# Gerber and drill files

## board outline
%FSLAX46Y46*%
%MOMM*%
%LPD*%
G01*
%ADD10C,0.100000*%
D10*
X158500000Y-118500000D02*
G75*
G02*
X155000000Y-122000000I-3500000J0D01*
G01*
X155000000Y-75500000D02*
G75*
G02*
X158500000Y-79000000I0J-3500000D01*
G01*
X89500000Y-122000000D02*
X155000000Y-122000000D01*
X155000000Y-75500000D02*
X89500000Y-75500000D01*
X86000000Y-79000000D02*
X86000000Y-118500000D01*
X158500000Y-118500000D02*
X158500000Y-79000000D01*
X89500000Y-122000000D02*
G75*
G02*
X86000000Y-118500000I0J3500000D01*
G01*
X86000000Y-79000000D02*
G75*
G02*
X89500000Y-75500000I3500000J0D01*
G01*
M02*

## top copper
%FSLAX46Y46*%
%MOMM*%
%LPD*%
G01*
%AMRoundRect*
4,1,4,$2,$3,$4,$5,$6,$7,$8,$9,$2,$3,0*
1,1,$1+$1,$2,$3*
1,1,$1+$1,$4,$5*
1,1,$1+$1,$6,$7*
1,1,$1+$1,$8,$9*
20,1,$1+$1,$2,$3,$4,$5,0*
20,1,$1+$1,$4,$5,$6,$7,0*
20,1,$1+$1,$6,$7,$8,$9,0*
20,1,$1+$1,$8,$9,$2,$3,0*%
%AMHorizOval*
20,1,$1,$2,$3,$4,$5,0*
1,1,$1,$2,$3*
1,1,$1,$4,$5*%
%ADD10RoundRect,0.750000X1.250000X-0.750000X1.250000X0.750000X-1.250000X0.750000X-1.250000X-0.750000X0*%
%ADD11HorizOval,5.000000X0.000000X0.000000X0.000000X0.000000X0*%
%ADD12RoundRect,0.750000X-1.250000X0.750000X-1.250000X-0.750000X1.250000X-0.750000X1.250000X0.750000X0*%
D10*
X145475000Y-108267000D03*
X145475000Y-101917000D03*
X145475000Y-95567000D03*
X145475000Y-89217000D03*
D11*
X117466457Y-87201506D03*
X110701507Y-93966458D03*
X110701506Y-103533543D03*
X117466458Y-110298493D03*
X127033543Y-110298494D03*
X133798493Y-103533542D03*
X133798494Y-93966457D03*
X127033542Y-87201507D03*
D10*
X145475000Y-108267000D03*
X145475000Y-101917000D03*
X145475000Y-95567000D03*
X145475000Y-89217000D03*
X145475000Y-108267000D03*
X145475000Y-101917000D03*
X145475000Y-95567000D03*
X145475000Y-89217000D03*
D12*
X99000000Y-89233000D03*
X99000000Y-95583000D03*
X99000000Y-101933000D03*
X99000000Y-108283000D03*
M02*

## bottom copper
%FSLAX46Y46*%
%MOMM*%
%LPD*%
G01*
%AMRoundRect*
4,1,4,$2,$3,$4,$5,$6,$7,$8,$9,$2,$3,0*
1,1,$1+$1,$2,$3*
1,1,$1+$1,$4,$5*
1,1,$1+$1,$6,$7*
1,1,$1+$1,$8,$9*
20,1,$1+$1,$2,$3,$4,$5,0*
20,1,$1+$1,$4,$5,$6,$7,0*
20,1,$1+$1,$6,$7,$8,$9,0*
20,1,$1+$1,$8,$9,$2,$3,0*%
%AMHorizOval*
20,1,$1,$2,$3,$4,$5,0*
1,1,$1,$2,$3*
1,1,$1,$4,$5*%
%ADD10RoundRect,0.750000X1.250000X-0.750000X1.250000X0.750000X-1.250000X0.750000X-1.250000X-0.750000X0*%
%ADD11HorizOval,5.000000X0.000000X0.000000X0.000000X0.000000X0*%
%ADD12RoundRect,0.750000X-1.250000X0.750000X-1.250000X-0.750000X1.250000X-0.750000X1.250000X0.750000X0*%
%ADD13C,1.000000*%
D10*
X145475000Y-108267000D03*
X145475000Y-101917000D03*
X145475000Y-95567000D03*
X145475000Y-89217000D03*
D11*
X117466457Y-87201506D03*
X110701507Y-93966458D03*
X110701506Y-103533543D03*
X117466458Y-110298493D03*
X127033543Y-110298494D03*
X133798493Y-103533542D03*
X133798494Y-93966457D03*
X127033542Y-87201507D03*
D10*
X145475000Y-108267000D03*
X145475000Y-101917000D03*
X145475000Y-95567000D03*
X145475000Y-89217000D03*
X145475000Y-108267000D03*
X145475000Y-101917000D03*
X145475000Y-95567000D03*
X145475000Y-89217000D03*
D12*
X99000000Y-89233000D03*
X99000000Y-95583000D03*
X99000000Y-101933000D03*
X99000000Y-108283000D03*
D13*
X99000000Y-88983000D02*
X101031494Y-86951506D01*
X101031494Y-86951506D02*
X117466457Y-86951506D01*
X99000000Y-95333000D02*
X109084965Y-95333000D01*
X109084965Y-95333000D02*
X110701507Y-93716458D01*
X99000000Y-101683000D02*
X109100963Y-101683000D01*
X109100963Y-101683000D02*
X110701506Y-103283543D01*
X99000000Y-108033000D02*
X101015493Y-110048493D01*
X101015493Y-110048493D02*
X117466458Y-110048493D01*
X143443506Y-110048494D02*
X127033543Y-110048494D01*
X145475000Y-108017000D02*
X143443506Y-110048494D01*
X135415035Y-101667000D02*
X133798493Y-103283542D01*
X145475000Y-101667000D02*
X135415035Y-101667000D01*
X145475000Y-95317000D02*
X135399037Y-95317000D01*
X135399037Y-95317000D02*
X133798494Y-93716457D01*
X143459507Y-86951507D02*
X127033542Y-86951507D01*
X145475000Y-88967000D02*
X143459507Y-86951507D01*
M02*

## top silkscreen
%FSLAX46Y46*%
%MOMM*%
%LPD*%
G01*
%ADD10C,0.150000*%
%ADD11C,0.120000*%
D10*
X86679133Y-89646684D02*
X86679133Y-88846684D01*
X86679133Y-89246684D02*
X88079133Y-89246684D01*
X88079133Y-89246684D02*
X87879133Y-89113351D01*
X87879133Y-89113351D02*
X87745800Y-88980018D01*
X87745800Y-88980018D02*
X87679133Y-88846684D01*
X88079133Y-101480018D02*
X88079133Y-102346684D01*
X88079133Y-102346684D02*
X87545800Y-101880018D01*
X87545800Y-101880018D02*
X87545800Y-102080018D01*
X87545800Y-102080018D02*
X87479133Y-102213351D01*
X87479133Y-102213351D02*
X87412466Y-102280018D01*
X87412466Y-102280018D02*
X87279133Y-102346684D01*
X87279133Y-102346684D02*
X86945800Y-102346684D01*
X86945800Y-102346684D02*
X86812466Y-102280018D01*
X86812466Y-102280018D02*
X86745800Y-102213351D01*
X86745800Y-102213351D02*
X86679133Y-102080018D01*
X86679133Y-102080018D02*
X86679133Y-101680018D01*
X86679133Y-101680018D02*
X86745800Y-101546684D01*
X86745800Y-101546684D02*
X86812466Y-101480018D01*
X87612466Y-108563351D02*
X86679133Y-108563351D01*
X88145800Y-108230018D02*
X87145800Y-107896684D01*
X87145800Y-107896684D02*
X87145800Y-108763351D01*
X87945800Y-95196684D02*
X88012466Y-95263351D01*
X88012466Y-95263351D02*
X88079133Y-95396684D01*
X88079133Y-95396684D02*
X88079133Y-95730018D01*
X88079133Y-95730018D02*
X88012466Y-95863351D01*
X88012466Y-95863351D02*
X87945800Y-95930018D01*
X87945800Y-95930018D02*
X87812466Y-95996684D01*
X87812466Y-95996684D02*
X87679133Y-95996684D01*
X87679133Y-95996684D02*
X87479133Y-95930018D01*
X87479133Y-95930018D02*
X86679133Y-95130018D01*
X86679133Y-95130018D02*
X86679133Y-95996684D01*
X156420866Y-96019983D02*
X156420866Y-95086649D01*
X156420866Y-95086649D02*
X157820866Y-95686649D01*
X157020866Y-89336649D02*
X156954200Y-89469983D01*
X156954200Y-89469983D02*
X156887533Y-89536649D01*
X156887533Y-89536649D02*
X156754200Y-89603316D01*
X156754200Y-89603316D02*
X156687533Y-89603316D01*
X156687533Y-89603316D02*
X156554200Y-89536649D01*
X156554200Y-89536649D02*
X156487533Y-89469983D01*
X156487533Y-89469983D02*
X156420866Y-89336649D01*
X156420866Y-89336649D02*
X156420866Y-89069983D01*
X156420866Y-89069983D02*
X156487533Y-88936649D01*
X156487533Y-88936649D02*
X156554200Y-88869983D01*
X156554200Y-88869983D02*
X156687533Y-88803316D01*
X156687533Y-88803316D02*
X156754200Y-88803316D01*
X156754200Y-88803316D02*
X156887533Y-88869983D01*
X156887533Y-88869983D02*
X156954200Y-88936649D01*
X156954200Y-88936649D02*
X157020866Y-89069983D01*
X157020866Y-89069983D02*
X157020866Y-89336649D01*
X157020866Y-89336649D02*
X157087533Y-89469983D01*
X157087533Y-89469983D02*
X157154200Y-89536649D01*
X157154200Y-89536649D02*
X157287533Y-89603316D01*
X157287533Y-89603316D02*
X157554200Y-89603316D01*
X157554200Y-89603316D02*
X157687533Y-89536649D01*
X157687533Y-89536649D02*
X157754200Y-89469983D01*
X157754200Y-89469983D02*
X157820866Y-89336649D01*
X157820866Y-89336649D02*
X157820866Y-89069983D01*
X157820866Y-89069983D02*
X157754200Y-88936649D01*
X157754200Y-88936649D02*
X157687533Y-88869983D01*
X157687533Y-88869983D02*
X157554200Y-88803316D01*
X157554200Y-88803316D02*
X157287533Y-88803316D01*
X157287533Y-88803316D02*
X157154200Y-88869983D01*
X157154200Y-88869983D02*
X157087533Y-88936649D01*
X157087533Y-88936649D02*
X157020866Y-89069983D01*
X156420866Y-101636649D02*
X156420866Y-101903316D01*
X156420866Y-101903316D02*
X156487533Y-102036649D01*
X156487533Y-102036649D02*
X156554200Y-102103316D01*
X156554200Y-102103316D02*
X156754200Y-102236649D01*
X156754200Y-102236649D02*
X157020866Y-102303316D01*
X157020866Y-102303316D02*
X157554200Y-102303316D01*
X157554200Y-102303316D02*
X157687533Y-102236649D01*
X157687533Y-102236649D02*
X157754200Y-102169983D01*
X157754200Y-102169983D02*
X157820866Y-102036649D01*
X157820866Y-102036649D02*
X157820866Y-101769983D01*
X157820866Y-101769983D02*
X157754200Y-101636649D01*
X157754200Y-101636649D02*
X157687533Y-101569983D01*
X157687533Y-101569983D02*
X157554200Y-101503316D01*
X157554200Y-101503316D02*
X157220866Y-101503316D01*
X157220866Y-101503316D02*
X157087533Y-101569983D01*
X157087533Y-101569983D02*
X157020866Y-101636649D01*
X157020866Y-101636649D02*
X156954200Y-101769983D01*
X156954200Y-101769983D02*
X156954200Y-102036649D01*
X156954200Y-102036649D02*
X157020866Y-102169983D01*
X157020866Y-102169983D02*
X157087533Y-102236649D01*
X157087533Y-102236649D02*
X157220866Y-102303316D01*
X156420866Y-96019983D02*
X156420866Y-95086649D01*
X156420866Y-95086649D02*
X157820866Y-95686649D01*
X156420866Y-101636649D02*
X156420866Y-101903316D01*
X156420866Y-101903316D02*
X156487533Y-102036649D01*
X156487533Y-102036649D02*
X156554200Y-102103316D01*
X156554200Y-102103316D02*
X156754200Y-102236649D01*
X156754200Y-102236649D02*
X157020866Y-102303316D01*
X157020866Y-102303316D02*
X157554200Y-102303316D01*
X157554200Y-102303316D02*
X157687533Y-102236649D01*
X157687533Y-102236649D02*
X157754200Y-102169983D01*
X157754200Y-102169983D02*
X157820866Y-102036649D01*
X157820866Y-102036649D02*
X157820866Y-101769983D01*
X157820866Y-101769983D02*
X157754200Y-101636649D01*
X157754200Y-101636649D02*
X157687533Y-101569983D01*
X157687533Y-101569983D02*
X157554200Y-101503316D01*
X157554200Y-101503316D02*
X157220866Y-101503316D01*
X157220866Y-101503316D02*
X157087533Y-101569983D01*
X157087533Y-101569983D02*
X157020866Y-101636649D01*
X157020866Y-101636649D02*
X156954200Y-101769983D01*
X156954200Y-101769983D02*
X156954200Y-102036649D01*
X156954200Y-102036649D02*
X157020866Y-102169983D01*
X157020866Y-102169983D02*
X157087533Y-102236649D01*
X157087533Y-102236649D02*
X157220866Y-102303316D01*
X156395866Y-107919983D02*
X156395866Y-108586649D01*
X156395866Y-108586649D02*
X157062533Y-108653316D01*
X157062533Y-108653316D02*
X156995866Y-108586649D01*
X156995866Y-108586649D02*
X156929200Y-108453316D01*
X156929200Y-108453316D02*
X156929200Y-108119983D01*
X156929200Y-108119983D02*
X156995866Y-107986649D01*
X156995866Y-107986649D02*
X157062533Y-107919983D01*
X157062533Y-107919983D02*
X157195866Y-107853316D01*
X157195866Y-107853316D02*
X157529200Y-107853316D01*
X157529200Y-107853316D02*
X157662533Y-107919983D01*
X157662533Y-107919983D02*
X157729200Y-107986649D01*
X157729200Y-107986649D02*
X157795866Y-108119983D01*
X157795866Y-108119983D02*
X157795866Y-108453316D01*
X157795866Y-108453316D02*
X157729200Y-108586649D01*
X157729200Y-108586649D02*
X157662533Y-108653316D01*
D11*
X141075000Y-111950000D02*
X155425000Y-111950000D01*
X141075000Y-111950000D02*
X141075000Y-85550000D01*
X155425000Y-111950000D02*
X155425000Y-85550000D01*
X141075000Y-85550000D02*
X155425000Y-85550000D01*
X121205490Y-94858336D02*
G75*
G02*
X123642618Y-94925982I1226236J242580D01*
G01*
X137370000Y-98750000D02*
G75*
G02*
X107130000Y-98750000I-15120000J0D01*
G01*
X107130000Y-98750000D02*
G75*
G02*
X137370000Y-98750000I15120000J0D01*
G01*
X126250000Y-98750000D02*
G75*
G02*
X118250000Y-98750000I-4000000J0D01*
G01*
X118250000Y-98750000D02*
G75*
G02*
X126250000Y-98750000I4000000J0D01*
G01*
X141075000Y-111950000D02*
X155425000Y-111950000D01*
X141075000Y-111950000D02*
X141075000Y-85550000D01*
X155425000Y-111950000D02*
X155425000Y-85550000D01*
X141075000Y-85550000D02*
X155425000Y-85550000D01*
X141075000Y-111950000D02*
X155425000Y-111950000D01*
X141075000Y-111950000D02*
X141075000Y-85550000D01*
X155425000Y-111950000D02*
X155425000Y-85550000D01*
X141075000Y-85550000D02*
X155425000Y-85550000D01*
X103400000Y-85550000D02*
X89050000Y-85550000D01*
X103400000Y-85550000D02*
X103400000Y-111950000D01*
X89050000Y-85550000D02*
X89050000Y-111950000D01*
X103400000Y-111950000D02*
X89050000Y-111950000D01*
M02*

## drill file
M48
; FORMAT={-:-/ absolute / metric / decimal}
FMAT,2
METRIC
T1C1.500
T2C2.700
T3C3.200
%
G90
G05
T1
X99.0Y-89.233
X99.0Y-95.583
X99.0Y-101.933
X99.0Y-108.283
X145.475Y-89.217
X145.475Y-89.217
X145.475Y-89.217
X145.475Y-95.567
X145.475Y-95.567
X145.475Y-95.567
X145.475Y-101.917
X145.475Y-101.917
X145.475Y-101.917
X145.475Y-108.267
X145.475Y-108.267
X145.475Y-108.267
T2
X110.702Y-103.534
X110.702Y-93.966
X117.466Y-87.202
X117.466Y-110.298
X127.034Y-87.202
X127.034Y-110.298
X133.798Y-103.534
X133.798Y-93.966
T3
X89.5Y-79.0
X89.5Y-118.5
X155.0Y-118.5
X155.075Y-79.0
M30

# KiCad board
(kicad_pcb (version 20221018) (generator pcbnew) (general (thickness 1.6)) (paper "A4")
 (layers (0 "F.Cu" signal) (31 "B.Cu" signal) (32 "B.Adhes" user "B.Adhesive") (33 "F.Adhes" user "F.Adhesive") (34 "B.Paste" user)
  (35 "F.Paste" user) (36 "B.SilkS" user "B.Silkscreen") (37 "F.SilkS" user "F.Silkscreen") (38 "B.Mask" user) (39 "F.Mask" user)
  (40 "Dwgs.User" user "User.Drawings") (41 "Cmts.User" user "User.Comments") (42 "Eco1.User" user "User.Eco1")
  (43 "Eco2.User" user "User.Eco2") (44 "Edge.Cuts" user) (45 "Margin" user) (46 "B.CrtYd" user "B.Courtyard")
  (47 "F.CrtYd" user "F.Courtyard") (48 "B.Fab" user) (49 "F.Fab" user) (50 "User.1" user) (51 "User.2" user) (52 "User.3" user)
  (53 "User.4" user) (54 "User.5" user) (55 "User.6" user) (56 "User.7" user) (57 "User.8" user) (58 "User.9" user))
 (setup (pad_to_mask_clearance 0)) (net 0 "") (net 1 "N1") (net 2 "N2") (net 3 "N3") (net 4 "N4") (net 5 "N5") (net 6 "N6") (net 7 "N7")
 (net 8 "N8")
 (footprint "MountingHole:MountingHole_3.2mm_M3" (layer "F.Cu") (at 89.5 118.5)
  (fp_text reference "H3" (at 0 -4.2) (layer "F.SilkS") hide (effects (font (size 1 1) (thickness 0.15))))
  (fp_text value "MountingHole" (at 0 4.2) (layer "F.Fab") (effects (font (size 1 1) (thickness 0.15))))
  (pad "" np_thru_hole circle (at 0 0) (size 3.2 3.2) (drill 3.2) (layers "*.Cu" "*.Mask")))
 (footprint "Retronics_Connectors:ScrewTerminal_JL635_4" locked (layer "F.Cu") (at 145.475 108.267 90)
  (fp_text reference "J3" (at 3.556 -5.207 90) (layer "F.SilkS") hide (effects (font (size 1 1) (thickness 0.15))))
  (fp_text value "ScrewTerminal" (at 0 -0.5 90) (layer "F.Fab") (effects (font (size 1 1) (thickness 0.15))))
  (fp_line (start -3.683 -4.4) (end -3.683 9.95) (stroke (width 0.12) (type solid)) (layer "F.SilkS"))
  (fp_line (start -3.683 -4.4) (end 22.717 -4.4) (stroke (width 0.12) (type solid)) (layer "F.SilkS"))
  (fp_line (start -3.683 9.95) (end 22.717 9.95) (stroke (width 0.12) (type solid)) (layer "F.SilkS"))
  (fp_line (start 22.717 -4.4) (end 22.717 9.95) (stroke (width 0.12) (type solid)) (layer "F.SilkS"))
  (pad "1" thru_hole roundrect locked (at 0 0 90) (size 3 4) (drill 1.5) (layers "*.Cu" "*.Mask") (roundrect_rratio 0.25) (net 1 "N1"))
  (pad "2" thru_hole roundrect locked (at 6.35 0 90) (size 3 4) (drill 1.5) (layers "*.Cu" "*.Mask") (roundrect_rratio 0.25) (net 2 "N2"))
  (pad "3" thru_hole roundrect locked (at 12.7 0 90) (size 3 4) (drill 1.5) (layers "*.Cu" "*.Mask") (roundrect_rratio 0.25) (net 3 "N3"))
  (pad "4" thru_hole roundrect locked (at 19.05 0 90) (size 3 4) (drill 1.5) (layers "*.Cu" "*.Mask") (roundrect_rratio 0.25) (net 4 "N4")))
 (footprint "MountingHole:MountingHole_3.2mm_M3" (layer "F.Cu") (at 155 118.5)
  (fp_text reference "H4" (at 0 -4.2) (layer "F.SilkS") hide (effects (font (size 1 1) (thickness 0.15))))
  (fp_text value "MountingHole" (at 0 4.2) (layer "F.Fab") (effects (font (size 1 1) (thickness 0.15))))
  (pad "" np_thru_hole circle (at 0 0) (size 3.2 3.2) (drill 3.2) (layers "*.Cu" "*.Mask")))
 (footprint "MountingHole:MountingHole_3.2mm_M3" (layer "F.Cu") (at 89.5 79)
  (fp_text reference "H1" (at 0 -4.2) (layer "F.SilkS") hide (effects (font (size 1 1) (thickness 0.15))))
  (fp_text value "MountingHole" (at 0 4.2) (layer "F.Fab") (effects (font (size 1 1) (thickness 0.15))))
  (pad "" np_thru_hole circle (at 0 0) (size 3.2 3.2) (drill 3.2) (layers "*.Cu" "*.Mask")))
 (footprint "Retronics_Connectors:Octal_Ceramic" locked (layer "F.Cu") (at 122.25 98.75 22.5)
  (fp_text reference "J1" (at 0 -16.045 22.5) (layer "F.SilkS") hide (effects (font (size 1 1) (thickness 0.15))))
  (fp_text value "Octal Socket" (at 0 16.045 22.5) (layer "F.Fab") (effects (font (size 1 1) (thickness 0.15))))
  (fp_arc (start 0.524274 -3.995145) (mid 2.260212 -4.891133) (end 2.75 -3) (stroke (width 0.12) (type solid)) (layer "F.SilkS"))
  (fp_circle (center 0 0) (end 0 15.12) (stroke (width 0.12) (type solid)) (fill none) (layer "F.SilkS"))
  (fp_circle (center 0 0) (end 4 0) (stroke (width 0.12) (type solid)) (fill none) (layer "F.SilkS"))
  (pad "1" thru_hole oval locked (at 0 -12.5 22.5) (size 5 5) (drill 2.7) (layers "*.Cu" "*.Mask") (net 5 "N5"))
  (pad "2" thru_hole oval locked (at -8.838834 -8.838834 22.5) (size 5 5) (drill 2.7) (layers "*.Cu" "*.Mask") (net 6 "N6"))
  (pad "3" thru_hole oval locked (at -12.5 0 22.5) (size 5 5) (drill 2.7) (layers "*.Cu" "*.Mask") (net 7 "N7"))
  (pad "4" thru_hole oval locked (at -8.838834 8.838834 22.5) (size 5 5) (drill 2.7) (layers "*.Cu" "*.Mask") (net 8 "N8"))
  (pad "5" thru_hole oval locked (at 0 12.5 22.5) (size 5 5) (drill 2.7) (layers "*.Cu" "*.Mask") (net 1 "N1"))
  (pad "6" thru_hole oval locked (at 8.838834 8.838834 22.5) (size 5 5) (drill 2.7) (layers "*.Cu" "*.Mask") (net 2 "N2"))
  (pad "7" thru_hole oval locked (at 12.5 0 22.5) (size 5 5) (drill 2.7) (layers "*.Cu" "*.Mask") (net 3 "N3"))
  (pad "8" thru_hole oval locked (at 8.838834 -8.838834 22.5) (size 5 5) (drill 2.7) (layers "*.Cu" "*.Mask") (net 4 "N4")))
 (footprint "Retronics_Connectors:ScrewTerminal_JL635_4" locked (layer "F.Cu") (at 145.475 108.267 90)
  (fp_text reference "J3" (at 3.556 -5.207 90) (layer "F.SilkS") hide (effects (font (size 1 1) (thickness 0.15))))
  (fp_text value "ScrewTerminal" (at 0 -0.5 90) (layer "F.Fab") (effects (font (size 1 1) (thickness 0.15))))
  (fp_line (start -3.683 -4.4) (end -3.683 9.95) (stroke (width 0.12) (type solid)) (layer "F.SilkS"))
  (fp_line (start -3.683 -4.4) (end 22.717 -4.4) (stroke (width 0.12) (type solid)) (layer "F.SilkS"))
  (fp_line (start -3.683 9.95) (end 22.717 9.95) (stroke (width 0.12) (type solid)) (layer "F.SilkS"))
  (fp_line (start 22.717 -4.4) (end 22.717 9.95) (stroke (width 0.12) (type solid)) (layer "F.SilkS"))
  (pad "1" thru_hole roundrect locked (at 0 0 90) (size 3 4) (drill 1.5) (layers "*.Cu" "*.Mask") (roundrect_rratio 0.25) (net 1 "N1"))
  (pad "2" thru_hole roundrect locked (at 6.35 0 90) (size 3 4) (drill 1.5) (layers "*.Cu" "*.Mask") (roundrect_rratio 0.25) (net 2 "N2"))
  (pad "3" thru_hole roundrect locked (at 12.7 0 90) (size 3 4) (drill 1.5) (layers "*.Cu" "*.Mask") (roundrect_rratio 0.25) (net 3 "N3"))
  (pad "4" thru_hole roundrect locked (at 19.05 0 90) (size 3 4) (drill 1.5) (layers "*.Cu" "*.Mask") (roundrect_rratio 0.25) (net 4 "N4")))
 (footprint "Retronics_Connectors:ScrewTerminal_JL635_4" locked (layer "F.Cu") (at 145.475 108.267 90)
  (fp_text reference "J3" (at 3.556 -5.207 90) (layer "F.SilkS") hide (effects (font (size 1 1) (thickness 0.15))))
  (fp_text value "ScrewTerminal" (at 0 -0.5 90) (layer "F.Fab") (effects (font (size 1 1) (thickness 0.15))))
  (fp_line (start -3.683 -4.4) (end -3.683 9.95) (stroke (width 0.12) (type solid)) (layer "F.SilkS"))
  (fp_line (start -3.683 -4.4) (end 22.717 -4.4) (stroke (width 0.12) (type solid)) (layer "F.SilkS"))
  (fp_line (start -3.683 9.95) (end 22.717 9.95) (stroke (width 0.12) (type solid)) (layer "F.SilkS"))
  (fp_line (start 22.717 -4.4) (end 22.717 9.95) (stroke (width 0.12) (type solid)) (layer "F.SilkS"))
  (pad "1" thru_hole roundrect locked (at 0 0 90) (size 3 4) (drill 1.5) (layers "*.Cu" "*.Mask") (roundrect_rratio 0.25) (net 1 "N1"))
  (pad "2" thru_hole roundrect locked (at 6.35 0 90) (size 3 4) (drill 1.5) (layers "*.Cu" "*.Mask") (roundrect_rratio 0.25) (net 2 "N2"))
  (pad "3" thru_hole roundrect locked (at 12.7 0 90) (size 3 4) (drill 1.5) (layers "*.Cu" "*.Mask") (roundrect_rratio 0.25) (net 3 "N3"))
  (pad "4" thru_hole roundrect locked (at 19.05 0 90) (size 3 4) (drill 1.5) (layers "*.Cu" "*.Mask") (roundrect_rratio 0.25) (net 4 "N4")))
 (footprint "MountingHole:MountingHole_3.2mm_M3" (layer "F.Cu") (at 155.075 79)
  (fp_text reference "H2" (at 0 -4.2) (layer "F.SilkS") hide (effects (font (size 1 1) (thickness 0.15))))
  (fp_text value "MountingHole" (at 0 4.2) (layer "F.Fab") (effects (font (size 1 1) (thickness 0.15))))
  (pad "" np_thru_hole circle (at 0 0) (size 3.2 3.2) (drill 3.2) (layers "*.Cu" "*.Mask")))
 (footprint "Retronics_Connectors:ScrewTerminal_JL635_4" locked (layer "F.Cu") (at 99 89.233 -90)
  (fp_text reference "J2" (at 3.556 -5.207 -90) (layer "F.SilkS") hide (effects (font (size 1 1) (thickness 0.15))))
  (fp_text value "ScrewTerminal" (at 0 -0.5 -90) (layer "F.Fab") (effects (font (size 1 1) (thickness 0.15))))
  (fp_line (start -3.683 -4.4) (end -3.683 9.95) (stroke (width 0.12) (type solid)) (layer "F.SilkS"))
  (fp_line (start -3.683 -4.4) (end 22.717 -4.4) (stroke (width 0.12) (type solid)) (layer "F.SilkS"))
  (fp_line (start -3.683 9.95) (end 22.717 9.95) (stroke (width 0.12) (type solid)) (layer "F.SilkS"))
  (fp_line (start 22.717 -4.4) (end 22.717 9.95) (stroke (width 0.12) (type solid)) (layer "F.SilkS"))
  (pad "1" thru_hole roundrect locked (at 0 0 270) (size 3 4) (drill 1.5) (layers "*.Cu" "*.Mask") (roundrect_rratio 0.25) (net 5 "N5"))
  (pad "2" thru_hole roundrect locked (at 6.35 0 270) (size 3 4) (drill 1.5) (layers "*.Cu" "*.Mask") (roundrect_rratio 0.25) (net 6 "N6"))
  (pad "3" thru_hole roundrect locked (at 12.7 0 270) (size 3 4) (drill 1.5) (layers "*.Cu" "*.Mask") (roundrect_rratio 0.25) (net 7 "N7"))
  (pad "4" thru_hole roundrect locked (at 19.05 0 270) (size 3 4) (drill 1.5) (layers "*.Cu" "*.Mask") (roundrect_rratio 0.25) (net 8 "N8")))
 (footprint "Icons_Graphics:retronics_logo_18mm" (layer "B.Cu") (at 122.233221 95.5 180)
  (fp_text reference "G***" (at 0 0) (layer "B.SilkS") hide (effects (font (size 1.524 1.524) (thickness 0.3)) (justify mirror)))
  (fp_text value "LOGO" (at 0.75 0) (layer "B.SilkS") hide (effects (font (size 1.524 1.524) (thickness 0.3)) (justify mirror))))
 (gr_arc (start 158.5 118.5) (mid 157.474874 120.974874) (end 155 122) (stroke (width 0.1) (type default)) (layer "Edge.Cuts"))
 (gr_arc (start 155 75.5) (mid 157.474874 76.525126) (end 158.5 79) (stroke (width 0.1) (type default)) (layer "Edge.Cuts"))
 (gr_line (start 89.5 122) (end 155 122) (stroke (width 0.1) (type default)) (layer "Edge.Cuts"))
 (gr_line (start 155 75.5) (end 89.5 75.5) (stroke (width 0.1) (type default)) (layer "Edge.Cuts"))
 (gr_line (start 86 79) (end 86 118.5) (stroke (width 0.1) (type default)) (layer "Edge.Cuts"))
 (gr_line (start 158.5 118.5) (end 158.5 79) (stroke (width 0.1) (type default)) (layer "Edge.Cuts"))
 (gr_arc (start 89.5 122) (mid 87.025126 120.974874) (end 86 118.5) (stroke (width 0.1) (type default)) (layer "Edge.Cuts"))
 (gr_arc (start 86 79) (mid 87.025126 76.525126) (end 89.5 75.5) (stroke (width 0.1) (type default)) (layer "Edge.Cuts"))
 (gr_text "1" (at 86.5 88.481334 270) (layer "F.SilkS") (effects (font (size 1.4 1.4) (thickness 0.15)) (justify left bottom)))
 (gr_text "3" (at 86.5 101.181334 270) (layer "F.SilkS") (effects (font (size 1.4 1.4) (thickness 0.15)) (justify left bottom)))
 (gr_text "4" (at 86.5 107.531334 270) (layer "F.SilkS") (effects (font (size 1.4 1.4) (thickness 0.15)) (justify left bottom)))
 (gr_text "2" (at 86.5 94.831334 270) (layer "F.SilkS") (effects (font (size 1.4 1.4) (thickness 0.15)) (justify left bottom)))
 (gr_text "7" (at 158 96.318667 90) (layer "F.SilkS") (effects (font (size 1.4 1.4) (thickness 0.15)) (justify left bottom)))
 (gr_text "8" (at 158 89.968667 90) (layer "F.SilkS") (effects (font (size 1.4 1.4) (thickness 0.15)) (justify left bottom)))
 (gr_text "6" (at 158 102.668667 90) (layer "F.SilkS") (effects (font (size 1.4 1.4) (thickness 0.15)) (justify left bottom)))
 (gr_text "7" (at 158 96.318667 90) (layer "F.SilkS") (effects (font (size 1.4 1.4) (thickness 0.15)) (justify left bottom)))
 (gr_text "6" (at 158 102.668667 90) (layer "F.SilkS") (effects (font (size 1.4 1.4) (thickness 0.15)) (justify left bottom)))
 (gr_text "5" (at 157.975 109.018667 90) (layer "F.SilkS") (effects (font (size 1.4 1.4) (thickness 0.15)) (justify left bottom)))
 (segment (start 99 88.983) (end 101.031494 86.951506) (width 1) (layer "B.Cu") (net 5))
 (segment (start 101.031494 86.951506) (end 117.466457 86.951506) (width 1) (layer "B.Cu") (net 5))
 (segment (start 99 95.333) (end 109.084965 95.333) (width 1) (layer "B.Cu") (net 6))
 (segment (start 109.084965 95.333) (end 110.701507 93.716458) (width 1) (layer "B.Cu") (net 6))
 (segment (start 99 101.683) (end 109.100963 101.683) (width 1) (layer "B.Cu") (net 7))
 (segment (start 109.100963 101.683) (end 110.701506 103.283543) (width 1) (layer "B.Cu") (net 7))
 (segment (start 99 108.033) (end 101.015493 110.048493) (width 1) (layer "B.Cu") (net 8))
 (segment (start 101.015493 110.048493) (end 117.466458 110.048493) (width 1) (layer "B.Cu") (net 8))
 (segment (start 143.443506 110.048494) (end 127.033543 110.048494) (width 1) (layer "B.Cu") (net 1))
 (segment (start 145.475 108.017) (end 143.443506 110.048494) (width 1) (layer "B.Cu") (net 1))
 (segment (start 135.415035 101.667) (end 133.798493 103.283542) (width 1) (layer "B.Cu") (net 2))
 (segment (start 145.475 101.667) (end 135.415035 101.667) (width 1) (layer "B.Cu") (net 2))
 (segment (start 145.475 95.317) (end 135.399037 95.317) (width 1) (layer "B.Cu") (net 3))
 (segment (start 135.399037 95.317) (end 133.798494 93.716457) (width 1) (layer "B.Cu") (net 3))
 (segment (start 143.459507 86.951507) (end 127.033542 86.951507) (width 1) (layer "B.Cu") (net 4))
 (segment (start 145.475 88.967) (end 143.459507 86.951507) (width 1) (layer "B.Cu") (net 4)))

